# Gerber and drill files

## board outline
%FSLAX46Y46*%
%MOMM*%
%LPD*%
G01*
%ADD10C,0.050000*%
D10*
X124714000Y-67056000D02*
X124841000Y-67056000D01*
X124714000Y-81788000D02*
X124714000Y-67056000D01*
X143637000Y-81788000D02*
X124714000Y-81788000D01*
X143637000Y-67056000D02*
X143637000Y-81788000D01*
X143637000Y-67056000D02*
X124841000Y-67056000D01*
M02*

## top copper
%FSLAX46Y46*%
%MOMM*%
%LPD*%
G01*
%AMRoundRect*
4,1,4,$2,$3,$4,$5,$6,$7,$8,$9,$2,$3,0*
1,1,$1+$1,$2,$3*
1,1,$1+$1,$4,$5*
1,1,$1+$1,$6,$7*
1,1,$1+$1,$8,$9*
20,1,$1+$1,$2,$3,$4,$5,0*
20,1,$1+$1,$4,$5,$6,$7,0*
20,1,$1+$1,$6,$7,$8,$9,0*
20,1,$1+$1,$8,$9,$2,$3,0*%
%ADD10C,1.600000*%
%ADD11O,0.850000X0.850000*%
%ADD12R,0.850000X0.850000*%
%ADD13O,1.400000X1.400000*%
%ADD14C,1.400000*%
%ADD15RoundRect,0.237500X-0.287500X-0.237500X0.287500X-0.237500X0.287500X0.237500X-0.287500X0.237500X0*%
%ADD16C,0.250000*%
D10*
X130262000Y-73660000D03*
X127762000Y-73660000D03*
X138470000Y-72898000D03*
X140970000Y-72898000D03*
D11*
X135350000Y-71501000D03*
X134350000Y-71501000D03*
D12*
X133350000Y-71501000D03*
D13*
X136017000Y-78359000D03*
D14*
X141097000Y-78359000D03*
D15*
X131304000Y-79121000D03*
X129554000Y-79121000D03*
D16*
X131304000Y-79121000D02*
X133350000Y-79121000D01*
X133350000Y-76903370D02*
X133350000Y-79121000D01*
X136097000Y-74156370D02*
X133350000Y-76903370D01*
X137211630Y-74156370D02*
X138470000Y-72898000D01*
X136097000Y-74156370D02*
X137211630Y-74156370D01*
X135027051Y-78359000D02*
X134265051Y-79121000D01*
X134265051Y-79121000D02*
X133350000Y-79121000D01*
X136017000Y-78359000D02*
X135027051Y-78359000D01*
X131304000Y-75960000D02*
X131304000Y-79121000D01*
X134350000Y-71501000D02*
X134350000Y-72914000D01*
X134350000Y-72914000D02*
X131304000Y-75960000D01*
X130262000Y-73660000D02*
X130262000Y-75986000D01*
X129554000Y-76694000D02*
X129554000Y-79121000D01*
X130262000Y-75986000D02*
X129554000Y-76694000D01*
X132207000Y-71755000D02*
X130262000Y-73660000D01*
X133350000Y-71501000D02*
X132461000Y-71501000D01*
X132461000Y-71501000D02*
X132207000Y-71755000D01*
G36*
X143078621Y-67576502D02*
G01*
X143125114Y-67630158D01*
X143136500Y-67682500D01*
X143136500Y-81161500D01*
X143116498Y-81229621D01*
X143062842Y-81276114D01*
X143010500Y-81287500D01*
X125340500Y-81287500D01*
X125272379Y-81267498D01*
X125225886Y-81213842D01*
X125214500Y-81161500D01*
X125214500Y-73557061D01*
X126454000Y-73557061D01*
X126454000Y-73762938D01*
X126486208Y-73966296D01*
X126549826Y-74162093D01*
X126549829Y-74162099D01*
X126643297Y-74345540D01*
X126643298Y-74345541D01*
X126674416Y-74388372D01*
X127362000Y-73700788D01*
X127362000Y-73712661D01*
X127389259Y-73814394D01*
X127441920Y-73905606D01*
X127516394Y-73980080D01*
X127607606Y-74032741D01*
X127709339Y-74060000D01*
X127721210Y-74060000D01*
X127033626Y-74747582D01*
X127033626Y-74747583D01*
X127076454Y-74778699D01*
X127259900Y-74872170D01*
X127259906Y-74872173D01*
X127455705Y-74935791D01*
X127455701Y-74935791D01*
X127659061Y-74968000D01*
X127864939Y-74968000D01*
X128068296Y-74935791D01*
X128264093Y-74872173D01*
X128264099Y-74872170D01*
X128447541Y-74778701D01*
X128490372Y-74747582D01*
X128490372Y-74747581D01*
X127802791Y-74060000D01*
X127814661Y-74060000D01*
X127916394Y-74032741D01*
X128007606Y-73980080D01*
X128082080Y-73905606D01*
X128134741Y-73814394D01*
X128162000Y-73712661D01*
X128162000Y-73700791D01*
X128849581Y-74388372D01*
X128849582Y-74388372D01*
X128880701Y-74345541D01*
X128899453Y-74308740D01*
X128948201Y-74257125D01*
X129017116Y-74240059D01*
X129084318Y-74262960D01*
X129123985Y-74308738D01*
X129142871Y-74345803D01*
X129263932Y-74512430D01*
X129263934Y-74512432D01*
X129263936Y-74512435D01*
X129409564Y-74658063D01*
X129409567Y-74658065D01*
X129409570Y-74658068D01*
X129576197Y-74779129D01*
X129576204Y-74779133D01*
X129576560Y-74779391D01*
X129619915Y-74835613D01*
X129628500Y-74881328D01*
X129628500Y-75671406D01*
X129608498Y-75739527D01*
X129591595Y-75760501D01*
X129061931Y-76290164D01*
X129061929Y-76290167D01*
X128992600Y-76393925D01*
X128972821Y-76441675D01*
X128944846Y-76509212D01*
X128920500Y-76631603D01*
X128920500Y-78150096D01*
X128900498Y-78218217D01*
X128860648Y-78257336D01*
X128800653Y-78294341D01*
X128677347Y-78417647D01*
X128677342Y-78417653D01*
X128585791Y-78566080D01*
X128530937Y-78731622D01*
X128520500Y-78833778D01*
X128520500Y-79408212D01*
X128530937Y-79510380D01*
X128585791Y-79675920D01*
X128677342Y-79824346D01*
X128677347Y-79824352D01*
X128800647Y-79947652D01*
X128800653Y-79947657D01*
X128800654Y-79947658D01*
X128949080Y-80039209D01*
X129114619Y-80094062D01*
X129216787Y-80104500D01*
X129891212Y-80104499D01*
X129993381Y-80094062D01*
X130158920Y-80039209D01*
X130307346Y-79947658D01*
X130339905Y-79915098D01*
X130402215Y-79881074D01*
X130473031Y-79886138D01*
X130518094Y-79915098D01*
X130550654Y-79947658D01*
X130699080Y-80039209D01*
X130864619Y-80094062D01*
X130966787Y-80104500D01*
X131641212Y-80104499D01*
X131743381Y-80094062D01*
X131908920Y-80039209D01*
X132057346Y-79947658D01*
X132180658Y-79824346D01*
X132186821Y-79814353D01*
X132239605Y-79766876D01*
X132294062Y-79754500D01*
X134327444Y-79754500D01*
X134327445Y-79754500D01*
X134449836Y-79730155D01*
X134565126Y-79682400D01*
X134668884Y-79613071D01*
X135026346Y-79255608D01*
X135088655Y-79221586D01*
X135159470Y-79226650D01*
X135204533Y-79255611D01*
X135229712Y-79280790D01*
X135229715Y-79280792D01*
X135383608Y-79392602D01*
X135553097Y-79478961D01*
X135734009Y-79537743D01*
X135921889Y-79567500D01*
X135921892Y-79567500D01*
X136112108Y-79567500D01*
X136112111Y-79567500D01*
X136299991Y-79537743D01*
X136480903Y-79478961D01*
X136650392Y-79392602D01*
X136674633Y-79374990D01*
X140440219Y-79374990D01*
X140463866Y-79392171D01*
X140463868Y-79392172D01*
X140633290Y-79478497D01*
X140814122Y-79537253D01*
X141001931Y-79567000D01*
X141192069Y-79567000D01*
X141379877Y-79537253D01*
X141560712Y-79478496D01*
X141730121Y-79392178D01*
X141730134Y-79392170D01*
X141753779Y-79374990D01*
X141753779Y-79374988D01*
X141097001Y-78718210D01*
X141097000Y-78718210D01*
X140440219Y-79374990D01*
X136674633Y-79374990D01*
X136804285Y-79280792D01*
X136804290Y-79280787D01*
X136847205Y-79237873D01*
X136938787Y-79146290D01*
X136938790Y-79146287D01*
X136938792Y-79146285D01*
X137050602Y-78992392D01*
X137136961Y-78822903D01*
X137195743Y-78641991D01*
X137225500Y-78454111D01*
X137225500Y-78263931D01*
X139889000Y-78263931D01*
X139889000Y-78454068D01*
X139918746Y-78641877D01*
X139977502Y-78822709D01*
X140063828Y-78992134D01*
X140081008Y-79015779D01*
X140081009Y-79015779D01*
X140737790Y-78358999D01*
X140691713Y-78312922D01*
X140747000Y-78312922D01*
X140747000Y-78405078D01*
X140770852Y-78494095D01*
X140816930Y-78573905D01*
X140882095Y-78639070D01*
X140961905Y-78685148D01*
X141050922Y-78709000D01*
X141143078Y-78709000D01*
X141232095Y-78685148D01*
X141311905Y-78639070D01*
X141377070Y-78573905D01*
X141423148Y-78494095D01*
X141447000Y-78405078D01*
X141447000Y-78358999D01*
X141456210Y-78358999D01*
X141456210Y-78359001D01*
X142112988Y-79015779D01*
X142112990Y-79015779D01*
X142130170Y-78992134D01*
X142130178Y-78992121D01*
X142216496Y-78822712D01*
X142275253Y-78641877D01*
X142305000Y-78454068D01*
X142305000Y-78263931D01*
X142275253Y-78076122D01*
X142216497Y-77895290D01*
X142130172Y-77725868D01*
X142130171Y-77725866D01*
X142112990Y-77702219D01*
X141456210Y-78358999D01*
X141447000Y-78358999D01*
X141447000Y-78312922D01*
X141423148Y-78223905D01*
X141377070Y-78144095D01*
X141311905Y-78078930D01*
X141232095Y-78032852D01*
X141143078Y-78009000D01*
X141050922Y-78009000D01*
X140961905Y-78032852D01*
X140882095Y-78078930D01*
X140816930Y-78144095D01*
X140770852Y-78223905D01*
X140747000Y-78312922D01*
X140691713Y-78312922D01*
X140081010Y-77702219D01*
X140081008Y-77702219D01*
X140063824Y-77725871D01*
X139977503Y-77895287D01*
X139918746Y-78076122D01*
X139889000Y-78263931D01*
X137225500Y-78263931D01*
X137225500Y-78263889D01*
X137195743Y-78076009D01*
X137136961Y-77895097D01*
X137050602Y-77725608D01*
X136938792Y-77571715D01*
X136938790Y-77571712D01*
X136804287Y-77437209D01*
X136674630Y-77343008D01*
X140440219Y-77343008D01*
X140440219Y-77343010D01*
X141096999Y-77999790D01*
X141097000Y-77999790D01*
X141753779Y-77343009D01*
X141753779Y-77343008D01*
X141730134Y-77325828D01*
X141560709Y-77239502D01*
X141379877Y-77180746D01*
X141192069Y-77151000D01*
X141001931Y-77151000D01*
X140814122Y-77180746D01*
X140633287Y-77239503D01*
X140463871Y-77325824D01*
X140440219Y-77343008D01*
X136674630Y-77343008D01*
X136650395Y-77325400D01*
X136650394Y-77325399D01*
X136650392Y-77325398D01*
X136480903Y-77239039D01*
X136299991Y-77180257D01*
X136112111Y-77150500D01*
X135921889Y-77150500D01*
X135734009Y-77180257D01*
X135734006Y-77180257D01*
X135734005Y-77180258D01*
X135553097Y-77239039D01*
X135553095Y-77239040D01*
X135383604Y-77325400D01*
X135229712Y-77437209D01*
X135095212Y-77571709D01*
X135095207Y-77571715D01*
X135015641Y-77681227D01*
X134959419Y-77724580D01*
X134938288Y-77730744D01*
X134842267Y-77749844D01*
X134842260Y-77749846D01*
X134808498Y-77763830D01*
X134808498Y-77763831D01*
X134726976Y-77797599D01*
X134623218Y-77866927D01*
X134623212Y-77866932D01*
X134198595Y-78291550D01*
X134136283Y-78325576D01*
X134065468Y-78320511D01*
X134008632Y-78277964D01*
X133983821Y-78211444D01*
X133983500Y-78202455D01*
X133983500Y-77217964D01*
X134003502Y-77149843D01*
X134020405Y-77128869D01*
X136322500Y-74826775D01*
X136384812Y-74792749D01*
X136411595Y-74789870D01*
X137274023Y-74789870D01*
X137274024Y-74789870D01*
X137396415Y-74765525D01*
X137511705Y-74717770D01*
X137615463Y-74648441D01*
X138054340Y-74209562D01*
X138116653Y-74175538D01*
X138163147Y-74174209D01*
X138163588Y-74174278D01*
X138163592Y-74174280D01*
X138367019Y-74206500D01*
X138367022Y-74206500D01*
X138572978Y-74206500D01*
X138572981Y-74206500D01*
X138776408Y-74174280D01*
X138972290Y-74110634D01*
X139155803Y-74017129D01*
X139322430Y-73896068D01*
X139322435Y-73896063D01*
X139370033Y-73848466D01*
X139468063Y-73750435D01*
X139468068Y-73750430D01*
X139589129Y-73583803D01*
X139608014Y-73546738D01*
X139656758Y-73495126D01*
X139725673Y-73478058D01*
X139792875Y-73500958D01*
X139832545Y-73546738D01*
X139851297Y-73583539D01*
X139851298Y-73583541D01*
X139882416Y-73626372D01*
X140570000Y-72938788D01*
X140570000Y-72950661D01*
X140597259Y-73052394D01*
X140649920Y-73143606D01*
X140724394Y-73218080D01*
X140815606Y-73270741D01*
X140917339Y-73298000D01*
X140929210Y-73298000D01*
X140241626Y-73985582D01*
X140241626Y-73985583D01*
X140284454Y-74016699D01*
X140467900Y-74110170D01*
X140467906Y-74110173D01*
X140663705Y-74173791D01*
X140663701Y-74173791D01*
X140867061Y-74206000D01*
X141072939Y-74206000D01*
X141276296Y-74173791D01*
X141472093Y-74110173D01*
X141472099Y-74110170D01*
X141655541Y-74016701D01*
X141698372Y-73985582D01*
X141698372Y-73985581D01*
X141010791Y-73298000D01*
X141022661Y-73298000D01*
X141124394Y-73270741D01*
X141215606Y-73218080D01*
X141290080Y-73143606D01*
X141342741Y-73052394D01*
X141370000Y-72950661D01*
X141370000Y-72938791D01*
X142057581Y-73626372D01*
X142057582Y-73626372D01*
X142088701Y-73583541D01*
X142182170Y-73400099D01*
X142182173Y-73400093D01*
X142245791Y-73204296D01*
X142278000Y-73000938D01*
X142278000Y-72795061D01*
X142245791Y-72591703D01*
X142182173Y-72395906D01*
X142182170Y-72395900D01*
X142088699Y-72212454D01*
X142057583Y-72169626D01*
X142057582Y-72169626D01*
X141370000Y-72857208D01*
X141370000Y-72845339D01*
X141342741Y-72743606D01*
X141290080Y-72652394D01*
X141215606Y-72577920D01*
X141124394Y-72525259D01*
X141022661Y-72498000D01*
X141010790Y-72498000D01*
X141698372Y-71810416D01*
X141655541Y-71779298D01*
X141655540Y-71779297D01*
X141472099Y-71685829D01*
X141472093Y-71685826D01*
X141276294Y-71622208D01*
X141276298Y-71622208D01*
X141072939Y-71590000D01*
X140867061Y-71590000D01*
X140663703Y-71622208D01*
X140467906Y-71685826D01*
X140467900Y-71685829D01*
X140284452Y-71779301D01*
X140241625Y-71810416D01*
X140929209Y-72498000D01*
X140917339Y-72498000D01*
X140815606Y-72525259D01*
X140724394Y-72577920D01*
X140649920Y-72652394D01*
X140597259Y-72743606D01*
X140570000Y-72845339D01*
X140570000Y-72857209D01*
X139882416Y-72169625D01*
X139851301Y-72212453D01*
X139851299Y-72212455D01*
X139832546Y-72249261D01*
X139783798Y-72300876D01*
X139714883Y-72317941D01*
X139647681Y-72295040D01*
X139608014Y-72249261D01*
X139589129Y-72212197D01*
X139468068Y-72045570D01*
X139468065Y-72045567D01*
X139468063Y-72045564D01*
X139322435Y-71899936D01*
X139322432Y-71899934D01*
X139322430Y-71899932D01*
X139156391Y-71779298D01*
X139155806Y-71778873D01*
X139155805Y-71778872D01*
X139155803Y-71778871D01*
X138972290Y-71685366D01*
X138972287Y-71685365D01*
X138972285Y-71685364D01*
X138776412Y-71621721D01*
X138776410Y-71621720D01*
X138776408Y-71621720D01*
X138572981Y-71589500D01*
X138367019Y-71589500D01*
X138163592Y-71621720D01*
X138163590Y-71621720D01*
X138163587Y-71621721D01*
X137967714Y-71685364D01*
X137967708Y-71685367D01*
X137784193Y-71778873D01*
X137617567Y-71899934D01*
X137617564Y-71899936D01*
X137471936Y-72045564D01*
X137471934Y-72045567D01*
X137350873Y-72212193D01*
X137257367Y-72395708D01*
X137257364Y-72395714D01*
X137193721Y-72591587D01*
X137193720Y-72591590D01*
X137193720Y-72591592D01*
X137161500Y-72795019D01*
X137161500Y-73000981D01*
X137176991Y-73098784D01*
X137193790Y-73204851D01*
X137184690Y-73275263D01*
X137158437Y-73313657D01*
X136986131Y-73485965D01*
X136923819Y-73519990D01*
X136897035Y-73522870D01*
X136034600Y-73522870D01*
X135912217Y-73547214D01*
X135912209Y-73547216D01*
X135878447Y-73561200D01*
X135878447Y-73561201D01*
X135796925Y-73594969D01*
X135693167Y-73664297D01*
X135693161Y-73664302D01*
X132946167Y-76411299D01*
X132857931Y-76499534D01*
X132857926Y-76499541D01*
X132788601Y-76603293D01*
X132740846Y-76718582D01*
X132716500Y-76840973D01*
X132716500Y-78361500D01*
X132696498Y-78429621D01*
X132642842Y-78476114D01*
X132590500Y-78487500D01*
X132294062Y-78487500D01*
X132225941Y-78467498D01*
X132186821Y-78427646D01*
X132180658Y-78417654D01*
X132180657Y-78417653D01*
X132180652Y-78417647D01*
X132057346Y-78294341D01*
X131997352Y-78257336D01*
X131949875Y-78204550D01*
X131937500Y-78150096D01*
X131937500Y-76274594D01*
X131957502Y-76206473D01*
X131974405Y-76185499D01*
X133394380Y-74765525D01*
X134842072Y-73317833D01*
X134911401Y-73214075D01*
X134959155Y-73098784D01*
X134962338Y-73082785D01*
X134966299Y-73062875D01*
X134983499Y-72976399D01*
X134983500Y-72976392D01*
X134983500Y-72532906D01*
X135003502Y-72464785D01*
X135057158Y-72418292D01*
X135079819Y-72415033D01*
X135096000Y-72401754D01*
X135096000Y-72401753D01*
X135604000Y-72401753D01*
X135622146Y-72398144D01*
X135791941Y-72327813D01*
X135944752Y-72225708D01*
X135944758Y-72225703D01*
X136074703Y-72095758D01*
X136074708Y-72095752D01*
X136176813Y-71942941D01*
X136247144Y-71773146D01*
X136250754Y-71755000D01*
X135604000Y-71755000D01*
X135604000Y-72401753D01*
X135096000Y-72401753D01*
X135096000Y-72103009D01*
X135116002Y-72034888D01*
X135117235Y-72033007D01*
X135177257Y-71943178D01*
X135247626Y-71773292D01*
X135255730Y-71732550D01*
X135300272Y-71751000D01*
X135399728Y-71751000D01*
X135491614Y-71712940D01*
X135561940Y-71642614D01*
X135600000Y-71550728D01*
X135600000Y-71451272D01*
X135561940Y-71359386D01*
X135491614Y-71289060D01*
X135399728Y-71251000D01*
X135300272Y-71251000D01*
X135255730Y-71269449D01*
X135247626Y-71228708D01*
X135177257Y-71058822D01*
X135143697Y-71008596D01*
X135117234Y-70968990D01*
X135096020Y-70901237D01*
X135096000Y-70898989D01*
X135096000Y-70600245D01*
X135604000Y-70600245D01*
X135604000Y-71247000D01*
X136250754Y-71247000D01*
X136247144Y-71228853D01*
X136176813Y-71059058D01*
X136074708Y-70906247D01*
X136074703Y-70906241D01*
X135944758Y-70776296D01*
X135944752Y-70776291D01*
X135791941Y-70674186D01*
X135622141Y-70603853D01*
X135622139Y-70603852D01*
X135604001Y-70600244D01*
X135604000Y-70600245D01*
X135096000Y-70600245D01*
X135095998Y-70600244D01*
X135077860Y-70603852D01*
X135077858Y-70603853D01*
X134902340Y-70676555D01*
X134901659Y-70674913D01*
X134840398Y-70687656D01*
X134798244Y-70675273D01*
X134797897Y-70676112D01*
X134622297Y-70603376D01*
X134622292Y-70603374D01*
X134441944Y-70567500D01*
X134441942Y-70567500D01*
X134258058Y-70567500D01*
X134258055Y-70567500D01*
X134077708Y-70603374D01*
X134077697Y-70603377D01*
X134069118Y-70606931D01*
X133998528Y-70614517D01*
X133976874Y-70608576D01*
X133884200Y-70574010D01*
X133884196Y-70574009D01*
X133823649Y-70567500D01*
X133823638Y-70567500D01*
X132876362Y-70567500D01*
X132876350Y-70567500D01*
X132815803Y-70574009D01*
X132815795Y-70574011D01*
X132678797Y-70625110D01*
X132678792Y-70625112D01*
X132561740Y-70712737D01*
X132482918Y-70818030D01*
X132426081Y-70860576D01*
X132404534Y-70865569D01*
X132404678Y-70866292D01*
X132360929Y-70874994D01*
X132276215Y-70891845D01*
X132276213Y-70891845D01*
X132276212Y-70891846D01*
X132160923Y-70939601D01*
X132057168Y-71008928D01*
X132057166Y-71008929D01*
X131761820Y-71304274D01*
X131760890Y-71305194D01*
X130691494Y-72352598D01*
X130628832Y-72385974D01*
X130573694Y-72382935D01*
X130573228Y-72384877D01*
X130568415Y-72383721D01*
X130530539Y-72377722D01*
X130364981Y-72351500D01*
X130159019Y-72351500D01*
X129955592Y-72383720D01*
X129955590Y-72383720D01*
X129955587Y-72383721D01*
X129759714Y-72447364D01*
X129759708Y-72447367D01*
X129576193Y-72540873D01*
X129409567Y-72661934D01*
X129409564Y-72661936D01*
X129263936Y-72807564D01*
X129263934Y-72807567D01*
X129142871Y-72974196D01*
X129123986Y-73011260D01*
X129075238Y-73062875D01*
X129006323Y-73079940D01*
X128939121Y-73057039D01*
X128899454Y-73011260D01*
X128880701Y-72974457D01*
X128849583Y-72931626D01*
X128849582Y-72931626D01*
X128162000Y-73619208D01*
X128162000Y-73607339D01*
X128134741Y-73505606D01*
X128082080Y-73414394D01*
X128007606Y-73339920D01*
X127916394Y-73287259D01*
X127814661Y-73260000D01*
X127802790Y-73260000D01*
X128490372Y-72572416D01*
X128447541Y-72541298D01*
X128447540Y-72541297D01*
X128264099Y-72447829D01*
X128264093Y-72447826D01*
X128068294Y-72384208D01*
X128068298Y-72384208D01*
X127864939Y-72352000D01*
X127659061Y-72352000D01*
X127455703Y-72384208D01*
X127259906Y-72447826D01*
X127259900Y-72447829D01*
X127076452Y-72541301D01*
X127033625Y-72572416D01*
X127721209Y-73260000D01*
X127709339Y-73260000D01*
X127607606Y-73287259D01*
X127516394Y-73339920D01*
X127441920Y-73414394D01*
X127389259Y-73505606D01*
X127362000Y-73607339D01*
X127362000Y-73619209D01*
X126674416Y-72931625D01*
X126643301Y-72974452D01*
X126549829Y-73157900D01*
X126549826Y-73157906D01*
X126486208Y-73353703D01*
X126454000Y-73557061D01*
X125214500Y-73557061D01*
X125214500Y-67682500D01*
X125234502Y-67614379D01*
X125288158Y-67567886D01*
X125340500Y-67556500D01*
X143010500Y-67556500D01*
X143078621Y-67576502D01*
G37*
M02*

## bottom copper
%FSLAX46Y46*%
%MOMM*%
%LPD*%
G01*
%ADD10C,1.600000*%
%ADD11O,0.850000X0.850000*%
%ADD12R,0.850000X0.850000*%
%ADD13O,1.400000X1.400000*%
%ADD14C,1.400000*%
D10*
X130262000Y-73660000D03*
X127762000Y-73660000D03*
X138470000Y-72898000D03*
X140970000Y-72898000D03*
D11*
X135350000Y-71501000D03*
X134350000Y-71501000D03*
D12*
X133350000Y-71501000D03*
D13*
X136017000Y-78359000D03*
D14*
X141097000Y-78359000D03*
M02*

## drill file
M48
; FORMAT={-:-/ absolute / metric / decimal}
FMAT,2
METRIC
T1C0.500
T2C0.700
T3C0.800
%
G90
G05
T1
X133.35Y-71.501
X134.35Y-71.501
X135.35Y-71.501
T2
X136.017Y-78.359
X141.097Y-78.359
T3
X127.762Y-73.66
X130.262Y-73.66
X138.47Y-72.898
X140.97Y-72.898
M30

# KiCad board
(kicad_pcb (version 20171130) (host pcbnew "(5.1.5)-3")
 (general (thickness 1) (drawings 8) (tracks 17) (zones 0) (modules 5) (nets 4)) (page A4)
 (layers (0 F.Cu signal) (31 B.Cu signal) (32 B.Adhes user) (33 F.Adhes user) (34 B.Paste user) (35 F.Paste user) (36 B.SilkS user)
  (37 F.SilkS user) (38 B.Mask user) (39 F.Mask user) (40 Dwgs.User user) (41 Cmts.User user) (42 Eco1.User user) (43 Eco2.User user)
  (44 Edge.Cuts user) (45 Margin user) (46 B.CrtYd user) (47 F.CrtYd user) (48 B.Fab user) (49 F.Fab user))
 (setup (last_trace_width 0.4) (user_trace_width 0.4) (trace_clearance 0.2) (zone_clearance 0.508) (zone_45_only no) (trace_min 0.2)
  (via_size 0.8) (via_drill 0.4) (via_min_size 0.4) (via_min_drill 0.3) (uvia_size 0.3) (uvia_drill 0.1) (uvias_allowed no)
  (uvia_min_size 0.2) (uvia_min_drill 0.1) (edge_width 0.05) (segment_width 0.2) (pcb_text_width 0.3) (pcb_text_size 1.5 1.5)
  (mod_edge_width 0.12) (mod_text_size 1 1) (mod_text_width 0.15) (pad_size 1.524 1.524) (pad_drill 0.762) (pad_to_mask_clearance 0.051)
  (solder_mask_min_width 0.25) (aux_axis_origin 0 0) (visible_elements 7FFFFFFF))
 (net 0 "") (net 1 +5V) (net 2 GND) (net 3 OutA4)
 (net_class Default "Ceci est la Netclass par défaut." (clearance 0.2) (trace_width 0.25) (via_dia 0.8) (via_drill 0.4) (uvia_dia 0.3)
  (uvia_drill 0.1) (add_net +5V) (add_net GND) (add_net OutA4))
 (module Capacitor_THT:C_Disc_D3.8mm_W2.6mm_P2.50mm (layer F.Cu) (at 127.762 73.66)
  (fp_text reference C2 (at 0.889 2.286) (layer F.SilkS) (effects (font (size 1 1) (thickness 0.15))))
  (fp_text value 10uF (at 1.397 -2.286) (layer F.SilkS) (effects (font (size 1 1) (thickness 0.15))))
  (pad 2 thru_hole circle (at 2.5 0) (size 1.6 1.6) (drill 0.8) (layers *.Cu *.Mask) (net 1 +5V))
  (pad 1 thru_hole circle (at 0 0) (size 1.6 1.6) (drill 0.8) (layers *.Cu *.Mask) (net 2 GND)))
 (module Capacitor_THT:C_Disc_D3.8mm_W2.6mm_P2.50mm (layer F.Cu) (at 140.97 72.898 180)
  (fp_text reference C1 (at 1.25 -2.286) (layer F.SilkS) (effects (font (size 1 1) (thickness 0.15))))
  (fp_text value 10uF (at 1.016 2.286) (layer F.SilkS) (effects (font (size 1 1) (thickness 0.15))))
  (pad 2 thru_hole circle (at 2.5 0 180) (size 1.6 1.6) (drill 0.8) (layers *.Cu *.Mask) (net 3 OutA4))
  (pad 1 thru_hole circle (at 0 0 180) (size 1.6 1.6) (drill 0.8) (layers *.Cu *.Mask) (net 2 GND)))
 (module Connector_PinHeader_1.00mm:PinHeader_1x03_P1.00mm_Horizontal (layer F.Cu) (at 133.35 71.501 90)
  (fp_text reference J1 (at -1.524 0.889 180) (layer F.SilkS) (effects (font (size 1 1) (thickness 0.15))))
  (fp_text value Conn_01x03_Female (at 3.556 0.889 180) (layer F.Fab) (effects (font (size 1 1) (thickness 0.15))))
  (pad 3 thru_hole oval (at 0 2 90) (size 0.85 0.85) (drill 0.5) (layers *.Cu *.Mask) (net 2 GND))
  (pad 2 thru_hole oval (at 0 1 90) (size 0.85 0.85) (drill 0.5) (layers *.Cu *.Mask) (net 3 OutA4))
  (pad 1 thru_hole rect (at 0 0 90) (size 0.85 0.85) (drill 0.5) (layers *.Cu *.Mask) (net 1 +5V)))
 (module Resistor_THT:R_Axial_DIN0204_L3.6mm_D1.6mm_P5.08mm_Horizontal (layer F.Cu) (at 141.097 78.359 180)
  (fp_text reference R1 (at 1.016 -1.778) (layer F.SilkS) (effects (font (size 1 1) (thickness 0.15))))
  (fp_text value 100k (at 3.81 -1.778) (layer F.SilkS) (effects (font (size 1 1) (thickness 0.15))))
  (pad 2 thru_hole oval (at 5.08 0 180) (size 1.4 1.4) (drill 0.7) (layers *.Cu *.Mask) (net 3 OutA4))
  (pad 1 thru_hole circle (at 0 0 180) (size 1.4 1.4) (drill 0.7) (layers *.Cu *.Mask) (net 2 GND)))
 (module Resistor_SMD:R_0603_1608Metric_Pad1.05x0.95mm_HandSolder (layer F.Cu) (at 130.429 79.121)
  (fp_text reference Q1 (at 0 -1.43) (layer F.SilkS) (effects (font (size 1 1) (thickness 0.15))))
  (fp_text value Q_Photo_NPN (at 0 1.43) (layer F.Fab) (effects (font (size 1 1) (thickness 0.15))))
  (pad 2 smd roundrect (at 0.875 0) (size 1.05 0.95) (layers F.Cu F.Paste F.Mask) (roundrect_rratio 0.25) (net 3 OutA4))
  (pad 1 smd roundrect (at -0.875 0) (size 1.05 0.95) (layers F.Cu F.Paste F.Mask) (roundrect_rratio 0.25) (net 1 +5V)))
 (gr_line (start 124.714 67.056) (end 124.841 67.056) (layer Edge.Cuts) (width 0.05))
 (gr_line (start 124.714 81.788) (end 124.714 67.056) (layer Edge.Cuts) (width 0.05))
 (gr_line (start 143.637 81.788) (end 124.714 81.788) (layer Edge.Cuts) (width 0.05))
 (gr_line (start 143.637 67.056) (end 143.637 81.788) (layer Edge.Cuts) (width 0.05))
 (gr_line (start 143.637 67.056) (end 124.841 67.056) (layer Edge.Cuts) (width 0.05))
 (segment (start 131.304 79.121) (end 133.35 79.121) (width 0.25) (layer F.Cu) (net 3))
 (segment (start 133.35 76.90337) (end 133.35 79.121) (width 0.25) (layer F.Cu) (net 3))
 (segment (start 136.097 74.15637) (end 133.35 76.90337) (width 0.25) (layer F.Cu) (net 3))
 (segment (start 137.21163 74.15637) (end 138.47 72.898) (width 0.25) (layer F.Cu) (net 3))
 (segment (start 136.097 74.15637) (end 137.21163 74.15637) (width 0.25) (layer F.Cu) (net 3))
 (segment (start 135.027051 78.359) (end 134.265051 79.121) (width 0.25) (layer F.Cu) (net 3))
 (segment (start 134.265051 79.121) (end 133.35 79.121) (width 0.25) (layer F.Cu) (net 3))
 (segment (start 136.017 78.359) (end 135.027051 78.359) (width 0.25) (layer F.Cu) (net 3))
 (segment (start 131.304 75.96) (end 131.304 79.121) (width 0.25) (layer F.Cu) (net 3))
 (segment (start 134.35 71.501) (end 134.35 72.914) (width 0.25) (layer F.Cu) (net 3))
 (segment (start 134.35 72.914) (end 131.304 75.96) (width 0.25) (layer F.Cu) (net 3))
 (segment (start 130.262 73.66) (end 130.262 75.986) (width 0.25) (layer F.Cu) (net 1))
 (segment (start 129.554 76.694) (end 129.554 79.121) (width 0.25) (layer F.Cu) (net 1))
 (segment (start 130.262 75.986) (end 129.554 76.694) (width 0.25) (layer F.Cu) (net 1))
 (segment (start 132.207 71.755) (end 130.262 73.66) (width 0.25) (layer F.Cu) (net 1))
 (segment (start 133.35 71.501) (end 132.461 71.501) (width 0.25) (layer F.Cu) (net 1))
 (segment (start 132.461 71.501) (end 132.207 71.755) (width 0.25) (layer F.Cu) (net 1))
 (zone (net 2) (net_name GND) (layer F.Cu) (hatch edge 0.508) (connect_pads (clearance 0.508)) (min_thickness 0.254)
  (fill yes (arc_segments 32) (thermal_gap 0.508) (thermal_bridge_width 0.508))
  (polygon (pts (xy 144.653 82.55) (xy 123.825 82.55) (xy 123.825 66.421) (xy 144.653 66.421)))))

